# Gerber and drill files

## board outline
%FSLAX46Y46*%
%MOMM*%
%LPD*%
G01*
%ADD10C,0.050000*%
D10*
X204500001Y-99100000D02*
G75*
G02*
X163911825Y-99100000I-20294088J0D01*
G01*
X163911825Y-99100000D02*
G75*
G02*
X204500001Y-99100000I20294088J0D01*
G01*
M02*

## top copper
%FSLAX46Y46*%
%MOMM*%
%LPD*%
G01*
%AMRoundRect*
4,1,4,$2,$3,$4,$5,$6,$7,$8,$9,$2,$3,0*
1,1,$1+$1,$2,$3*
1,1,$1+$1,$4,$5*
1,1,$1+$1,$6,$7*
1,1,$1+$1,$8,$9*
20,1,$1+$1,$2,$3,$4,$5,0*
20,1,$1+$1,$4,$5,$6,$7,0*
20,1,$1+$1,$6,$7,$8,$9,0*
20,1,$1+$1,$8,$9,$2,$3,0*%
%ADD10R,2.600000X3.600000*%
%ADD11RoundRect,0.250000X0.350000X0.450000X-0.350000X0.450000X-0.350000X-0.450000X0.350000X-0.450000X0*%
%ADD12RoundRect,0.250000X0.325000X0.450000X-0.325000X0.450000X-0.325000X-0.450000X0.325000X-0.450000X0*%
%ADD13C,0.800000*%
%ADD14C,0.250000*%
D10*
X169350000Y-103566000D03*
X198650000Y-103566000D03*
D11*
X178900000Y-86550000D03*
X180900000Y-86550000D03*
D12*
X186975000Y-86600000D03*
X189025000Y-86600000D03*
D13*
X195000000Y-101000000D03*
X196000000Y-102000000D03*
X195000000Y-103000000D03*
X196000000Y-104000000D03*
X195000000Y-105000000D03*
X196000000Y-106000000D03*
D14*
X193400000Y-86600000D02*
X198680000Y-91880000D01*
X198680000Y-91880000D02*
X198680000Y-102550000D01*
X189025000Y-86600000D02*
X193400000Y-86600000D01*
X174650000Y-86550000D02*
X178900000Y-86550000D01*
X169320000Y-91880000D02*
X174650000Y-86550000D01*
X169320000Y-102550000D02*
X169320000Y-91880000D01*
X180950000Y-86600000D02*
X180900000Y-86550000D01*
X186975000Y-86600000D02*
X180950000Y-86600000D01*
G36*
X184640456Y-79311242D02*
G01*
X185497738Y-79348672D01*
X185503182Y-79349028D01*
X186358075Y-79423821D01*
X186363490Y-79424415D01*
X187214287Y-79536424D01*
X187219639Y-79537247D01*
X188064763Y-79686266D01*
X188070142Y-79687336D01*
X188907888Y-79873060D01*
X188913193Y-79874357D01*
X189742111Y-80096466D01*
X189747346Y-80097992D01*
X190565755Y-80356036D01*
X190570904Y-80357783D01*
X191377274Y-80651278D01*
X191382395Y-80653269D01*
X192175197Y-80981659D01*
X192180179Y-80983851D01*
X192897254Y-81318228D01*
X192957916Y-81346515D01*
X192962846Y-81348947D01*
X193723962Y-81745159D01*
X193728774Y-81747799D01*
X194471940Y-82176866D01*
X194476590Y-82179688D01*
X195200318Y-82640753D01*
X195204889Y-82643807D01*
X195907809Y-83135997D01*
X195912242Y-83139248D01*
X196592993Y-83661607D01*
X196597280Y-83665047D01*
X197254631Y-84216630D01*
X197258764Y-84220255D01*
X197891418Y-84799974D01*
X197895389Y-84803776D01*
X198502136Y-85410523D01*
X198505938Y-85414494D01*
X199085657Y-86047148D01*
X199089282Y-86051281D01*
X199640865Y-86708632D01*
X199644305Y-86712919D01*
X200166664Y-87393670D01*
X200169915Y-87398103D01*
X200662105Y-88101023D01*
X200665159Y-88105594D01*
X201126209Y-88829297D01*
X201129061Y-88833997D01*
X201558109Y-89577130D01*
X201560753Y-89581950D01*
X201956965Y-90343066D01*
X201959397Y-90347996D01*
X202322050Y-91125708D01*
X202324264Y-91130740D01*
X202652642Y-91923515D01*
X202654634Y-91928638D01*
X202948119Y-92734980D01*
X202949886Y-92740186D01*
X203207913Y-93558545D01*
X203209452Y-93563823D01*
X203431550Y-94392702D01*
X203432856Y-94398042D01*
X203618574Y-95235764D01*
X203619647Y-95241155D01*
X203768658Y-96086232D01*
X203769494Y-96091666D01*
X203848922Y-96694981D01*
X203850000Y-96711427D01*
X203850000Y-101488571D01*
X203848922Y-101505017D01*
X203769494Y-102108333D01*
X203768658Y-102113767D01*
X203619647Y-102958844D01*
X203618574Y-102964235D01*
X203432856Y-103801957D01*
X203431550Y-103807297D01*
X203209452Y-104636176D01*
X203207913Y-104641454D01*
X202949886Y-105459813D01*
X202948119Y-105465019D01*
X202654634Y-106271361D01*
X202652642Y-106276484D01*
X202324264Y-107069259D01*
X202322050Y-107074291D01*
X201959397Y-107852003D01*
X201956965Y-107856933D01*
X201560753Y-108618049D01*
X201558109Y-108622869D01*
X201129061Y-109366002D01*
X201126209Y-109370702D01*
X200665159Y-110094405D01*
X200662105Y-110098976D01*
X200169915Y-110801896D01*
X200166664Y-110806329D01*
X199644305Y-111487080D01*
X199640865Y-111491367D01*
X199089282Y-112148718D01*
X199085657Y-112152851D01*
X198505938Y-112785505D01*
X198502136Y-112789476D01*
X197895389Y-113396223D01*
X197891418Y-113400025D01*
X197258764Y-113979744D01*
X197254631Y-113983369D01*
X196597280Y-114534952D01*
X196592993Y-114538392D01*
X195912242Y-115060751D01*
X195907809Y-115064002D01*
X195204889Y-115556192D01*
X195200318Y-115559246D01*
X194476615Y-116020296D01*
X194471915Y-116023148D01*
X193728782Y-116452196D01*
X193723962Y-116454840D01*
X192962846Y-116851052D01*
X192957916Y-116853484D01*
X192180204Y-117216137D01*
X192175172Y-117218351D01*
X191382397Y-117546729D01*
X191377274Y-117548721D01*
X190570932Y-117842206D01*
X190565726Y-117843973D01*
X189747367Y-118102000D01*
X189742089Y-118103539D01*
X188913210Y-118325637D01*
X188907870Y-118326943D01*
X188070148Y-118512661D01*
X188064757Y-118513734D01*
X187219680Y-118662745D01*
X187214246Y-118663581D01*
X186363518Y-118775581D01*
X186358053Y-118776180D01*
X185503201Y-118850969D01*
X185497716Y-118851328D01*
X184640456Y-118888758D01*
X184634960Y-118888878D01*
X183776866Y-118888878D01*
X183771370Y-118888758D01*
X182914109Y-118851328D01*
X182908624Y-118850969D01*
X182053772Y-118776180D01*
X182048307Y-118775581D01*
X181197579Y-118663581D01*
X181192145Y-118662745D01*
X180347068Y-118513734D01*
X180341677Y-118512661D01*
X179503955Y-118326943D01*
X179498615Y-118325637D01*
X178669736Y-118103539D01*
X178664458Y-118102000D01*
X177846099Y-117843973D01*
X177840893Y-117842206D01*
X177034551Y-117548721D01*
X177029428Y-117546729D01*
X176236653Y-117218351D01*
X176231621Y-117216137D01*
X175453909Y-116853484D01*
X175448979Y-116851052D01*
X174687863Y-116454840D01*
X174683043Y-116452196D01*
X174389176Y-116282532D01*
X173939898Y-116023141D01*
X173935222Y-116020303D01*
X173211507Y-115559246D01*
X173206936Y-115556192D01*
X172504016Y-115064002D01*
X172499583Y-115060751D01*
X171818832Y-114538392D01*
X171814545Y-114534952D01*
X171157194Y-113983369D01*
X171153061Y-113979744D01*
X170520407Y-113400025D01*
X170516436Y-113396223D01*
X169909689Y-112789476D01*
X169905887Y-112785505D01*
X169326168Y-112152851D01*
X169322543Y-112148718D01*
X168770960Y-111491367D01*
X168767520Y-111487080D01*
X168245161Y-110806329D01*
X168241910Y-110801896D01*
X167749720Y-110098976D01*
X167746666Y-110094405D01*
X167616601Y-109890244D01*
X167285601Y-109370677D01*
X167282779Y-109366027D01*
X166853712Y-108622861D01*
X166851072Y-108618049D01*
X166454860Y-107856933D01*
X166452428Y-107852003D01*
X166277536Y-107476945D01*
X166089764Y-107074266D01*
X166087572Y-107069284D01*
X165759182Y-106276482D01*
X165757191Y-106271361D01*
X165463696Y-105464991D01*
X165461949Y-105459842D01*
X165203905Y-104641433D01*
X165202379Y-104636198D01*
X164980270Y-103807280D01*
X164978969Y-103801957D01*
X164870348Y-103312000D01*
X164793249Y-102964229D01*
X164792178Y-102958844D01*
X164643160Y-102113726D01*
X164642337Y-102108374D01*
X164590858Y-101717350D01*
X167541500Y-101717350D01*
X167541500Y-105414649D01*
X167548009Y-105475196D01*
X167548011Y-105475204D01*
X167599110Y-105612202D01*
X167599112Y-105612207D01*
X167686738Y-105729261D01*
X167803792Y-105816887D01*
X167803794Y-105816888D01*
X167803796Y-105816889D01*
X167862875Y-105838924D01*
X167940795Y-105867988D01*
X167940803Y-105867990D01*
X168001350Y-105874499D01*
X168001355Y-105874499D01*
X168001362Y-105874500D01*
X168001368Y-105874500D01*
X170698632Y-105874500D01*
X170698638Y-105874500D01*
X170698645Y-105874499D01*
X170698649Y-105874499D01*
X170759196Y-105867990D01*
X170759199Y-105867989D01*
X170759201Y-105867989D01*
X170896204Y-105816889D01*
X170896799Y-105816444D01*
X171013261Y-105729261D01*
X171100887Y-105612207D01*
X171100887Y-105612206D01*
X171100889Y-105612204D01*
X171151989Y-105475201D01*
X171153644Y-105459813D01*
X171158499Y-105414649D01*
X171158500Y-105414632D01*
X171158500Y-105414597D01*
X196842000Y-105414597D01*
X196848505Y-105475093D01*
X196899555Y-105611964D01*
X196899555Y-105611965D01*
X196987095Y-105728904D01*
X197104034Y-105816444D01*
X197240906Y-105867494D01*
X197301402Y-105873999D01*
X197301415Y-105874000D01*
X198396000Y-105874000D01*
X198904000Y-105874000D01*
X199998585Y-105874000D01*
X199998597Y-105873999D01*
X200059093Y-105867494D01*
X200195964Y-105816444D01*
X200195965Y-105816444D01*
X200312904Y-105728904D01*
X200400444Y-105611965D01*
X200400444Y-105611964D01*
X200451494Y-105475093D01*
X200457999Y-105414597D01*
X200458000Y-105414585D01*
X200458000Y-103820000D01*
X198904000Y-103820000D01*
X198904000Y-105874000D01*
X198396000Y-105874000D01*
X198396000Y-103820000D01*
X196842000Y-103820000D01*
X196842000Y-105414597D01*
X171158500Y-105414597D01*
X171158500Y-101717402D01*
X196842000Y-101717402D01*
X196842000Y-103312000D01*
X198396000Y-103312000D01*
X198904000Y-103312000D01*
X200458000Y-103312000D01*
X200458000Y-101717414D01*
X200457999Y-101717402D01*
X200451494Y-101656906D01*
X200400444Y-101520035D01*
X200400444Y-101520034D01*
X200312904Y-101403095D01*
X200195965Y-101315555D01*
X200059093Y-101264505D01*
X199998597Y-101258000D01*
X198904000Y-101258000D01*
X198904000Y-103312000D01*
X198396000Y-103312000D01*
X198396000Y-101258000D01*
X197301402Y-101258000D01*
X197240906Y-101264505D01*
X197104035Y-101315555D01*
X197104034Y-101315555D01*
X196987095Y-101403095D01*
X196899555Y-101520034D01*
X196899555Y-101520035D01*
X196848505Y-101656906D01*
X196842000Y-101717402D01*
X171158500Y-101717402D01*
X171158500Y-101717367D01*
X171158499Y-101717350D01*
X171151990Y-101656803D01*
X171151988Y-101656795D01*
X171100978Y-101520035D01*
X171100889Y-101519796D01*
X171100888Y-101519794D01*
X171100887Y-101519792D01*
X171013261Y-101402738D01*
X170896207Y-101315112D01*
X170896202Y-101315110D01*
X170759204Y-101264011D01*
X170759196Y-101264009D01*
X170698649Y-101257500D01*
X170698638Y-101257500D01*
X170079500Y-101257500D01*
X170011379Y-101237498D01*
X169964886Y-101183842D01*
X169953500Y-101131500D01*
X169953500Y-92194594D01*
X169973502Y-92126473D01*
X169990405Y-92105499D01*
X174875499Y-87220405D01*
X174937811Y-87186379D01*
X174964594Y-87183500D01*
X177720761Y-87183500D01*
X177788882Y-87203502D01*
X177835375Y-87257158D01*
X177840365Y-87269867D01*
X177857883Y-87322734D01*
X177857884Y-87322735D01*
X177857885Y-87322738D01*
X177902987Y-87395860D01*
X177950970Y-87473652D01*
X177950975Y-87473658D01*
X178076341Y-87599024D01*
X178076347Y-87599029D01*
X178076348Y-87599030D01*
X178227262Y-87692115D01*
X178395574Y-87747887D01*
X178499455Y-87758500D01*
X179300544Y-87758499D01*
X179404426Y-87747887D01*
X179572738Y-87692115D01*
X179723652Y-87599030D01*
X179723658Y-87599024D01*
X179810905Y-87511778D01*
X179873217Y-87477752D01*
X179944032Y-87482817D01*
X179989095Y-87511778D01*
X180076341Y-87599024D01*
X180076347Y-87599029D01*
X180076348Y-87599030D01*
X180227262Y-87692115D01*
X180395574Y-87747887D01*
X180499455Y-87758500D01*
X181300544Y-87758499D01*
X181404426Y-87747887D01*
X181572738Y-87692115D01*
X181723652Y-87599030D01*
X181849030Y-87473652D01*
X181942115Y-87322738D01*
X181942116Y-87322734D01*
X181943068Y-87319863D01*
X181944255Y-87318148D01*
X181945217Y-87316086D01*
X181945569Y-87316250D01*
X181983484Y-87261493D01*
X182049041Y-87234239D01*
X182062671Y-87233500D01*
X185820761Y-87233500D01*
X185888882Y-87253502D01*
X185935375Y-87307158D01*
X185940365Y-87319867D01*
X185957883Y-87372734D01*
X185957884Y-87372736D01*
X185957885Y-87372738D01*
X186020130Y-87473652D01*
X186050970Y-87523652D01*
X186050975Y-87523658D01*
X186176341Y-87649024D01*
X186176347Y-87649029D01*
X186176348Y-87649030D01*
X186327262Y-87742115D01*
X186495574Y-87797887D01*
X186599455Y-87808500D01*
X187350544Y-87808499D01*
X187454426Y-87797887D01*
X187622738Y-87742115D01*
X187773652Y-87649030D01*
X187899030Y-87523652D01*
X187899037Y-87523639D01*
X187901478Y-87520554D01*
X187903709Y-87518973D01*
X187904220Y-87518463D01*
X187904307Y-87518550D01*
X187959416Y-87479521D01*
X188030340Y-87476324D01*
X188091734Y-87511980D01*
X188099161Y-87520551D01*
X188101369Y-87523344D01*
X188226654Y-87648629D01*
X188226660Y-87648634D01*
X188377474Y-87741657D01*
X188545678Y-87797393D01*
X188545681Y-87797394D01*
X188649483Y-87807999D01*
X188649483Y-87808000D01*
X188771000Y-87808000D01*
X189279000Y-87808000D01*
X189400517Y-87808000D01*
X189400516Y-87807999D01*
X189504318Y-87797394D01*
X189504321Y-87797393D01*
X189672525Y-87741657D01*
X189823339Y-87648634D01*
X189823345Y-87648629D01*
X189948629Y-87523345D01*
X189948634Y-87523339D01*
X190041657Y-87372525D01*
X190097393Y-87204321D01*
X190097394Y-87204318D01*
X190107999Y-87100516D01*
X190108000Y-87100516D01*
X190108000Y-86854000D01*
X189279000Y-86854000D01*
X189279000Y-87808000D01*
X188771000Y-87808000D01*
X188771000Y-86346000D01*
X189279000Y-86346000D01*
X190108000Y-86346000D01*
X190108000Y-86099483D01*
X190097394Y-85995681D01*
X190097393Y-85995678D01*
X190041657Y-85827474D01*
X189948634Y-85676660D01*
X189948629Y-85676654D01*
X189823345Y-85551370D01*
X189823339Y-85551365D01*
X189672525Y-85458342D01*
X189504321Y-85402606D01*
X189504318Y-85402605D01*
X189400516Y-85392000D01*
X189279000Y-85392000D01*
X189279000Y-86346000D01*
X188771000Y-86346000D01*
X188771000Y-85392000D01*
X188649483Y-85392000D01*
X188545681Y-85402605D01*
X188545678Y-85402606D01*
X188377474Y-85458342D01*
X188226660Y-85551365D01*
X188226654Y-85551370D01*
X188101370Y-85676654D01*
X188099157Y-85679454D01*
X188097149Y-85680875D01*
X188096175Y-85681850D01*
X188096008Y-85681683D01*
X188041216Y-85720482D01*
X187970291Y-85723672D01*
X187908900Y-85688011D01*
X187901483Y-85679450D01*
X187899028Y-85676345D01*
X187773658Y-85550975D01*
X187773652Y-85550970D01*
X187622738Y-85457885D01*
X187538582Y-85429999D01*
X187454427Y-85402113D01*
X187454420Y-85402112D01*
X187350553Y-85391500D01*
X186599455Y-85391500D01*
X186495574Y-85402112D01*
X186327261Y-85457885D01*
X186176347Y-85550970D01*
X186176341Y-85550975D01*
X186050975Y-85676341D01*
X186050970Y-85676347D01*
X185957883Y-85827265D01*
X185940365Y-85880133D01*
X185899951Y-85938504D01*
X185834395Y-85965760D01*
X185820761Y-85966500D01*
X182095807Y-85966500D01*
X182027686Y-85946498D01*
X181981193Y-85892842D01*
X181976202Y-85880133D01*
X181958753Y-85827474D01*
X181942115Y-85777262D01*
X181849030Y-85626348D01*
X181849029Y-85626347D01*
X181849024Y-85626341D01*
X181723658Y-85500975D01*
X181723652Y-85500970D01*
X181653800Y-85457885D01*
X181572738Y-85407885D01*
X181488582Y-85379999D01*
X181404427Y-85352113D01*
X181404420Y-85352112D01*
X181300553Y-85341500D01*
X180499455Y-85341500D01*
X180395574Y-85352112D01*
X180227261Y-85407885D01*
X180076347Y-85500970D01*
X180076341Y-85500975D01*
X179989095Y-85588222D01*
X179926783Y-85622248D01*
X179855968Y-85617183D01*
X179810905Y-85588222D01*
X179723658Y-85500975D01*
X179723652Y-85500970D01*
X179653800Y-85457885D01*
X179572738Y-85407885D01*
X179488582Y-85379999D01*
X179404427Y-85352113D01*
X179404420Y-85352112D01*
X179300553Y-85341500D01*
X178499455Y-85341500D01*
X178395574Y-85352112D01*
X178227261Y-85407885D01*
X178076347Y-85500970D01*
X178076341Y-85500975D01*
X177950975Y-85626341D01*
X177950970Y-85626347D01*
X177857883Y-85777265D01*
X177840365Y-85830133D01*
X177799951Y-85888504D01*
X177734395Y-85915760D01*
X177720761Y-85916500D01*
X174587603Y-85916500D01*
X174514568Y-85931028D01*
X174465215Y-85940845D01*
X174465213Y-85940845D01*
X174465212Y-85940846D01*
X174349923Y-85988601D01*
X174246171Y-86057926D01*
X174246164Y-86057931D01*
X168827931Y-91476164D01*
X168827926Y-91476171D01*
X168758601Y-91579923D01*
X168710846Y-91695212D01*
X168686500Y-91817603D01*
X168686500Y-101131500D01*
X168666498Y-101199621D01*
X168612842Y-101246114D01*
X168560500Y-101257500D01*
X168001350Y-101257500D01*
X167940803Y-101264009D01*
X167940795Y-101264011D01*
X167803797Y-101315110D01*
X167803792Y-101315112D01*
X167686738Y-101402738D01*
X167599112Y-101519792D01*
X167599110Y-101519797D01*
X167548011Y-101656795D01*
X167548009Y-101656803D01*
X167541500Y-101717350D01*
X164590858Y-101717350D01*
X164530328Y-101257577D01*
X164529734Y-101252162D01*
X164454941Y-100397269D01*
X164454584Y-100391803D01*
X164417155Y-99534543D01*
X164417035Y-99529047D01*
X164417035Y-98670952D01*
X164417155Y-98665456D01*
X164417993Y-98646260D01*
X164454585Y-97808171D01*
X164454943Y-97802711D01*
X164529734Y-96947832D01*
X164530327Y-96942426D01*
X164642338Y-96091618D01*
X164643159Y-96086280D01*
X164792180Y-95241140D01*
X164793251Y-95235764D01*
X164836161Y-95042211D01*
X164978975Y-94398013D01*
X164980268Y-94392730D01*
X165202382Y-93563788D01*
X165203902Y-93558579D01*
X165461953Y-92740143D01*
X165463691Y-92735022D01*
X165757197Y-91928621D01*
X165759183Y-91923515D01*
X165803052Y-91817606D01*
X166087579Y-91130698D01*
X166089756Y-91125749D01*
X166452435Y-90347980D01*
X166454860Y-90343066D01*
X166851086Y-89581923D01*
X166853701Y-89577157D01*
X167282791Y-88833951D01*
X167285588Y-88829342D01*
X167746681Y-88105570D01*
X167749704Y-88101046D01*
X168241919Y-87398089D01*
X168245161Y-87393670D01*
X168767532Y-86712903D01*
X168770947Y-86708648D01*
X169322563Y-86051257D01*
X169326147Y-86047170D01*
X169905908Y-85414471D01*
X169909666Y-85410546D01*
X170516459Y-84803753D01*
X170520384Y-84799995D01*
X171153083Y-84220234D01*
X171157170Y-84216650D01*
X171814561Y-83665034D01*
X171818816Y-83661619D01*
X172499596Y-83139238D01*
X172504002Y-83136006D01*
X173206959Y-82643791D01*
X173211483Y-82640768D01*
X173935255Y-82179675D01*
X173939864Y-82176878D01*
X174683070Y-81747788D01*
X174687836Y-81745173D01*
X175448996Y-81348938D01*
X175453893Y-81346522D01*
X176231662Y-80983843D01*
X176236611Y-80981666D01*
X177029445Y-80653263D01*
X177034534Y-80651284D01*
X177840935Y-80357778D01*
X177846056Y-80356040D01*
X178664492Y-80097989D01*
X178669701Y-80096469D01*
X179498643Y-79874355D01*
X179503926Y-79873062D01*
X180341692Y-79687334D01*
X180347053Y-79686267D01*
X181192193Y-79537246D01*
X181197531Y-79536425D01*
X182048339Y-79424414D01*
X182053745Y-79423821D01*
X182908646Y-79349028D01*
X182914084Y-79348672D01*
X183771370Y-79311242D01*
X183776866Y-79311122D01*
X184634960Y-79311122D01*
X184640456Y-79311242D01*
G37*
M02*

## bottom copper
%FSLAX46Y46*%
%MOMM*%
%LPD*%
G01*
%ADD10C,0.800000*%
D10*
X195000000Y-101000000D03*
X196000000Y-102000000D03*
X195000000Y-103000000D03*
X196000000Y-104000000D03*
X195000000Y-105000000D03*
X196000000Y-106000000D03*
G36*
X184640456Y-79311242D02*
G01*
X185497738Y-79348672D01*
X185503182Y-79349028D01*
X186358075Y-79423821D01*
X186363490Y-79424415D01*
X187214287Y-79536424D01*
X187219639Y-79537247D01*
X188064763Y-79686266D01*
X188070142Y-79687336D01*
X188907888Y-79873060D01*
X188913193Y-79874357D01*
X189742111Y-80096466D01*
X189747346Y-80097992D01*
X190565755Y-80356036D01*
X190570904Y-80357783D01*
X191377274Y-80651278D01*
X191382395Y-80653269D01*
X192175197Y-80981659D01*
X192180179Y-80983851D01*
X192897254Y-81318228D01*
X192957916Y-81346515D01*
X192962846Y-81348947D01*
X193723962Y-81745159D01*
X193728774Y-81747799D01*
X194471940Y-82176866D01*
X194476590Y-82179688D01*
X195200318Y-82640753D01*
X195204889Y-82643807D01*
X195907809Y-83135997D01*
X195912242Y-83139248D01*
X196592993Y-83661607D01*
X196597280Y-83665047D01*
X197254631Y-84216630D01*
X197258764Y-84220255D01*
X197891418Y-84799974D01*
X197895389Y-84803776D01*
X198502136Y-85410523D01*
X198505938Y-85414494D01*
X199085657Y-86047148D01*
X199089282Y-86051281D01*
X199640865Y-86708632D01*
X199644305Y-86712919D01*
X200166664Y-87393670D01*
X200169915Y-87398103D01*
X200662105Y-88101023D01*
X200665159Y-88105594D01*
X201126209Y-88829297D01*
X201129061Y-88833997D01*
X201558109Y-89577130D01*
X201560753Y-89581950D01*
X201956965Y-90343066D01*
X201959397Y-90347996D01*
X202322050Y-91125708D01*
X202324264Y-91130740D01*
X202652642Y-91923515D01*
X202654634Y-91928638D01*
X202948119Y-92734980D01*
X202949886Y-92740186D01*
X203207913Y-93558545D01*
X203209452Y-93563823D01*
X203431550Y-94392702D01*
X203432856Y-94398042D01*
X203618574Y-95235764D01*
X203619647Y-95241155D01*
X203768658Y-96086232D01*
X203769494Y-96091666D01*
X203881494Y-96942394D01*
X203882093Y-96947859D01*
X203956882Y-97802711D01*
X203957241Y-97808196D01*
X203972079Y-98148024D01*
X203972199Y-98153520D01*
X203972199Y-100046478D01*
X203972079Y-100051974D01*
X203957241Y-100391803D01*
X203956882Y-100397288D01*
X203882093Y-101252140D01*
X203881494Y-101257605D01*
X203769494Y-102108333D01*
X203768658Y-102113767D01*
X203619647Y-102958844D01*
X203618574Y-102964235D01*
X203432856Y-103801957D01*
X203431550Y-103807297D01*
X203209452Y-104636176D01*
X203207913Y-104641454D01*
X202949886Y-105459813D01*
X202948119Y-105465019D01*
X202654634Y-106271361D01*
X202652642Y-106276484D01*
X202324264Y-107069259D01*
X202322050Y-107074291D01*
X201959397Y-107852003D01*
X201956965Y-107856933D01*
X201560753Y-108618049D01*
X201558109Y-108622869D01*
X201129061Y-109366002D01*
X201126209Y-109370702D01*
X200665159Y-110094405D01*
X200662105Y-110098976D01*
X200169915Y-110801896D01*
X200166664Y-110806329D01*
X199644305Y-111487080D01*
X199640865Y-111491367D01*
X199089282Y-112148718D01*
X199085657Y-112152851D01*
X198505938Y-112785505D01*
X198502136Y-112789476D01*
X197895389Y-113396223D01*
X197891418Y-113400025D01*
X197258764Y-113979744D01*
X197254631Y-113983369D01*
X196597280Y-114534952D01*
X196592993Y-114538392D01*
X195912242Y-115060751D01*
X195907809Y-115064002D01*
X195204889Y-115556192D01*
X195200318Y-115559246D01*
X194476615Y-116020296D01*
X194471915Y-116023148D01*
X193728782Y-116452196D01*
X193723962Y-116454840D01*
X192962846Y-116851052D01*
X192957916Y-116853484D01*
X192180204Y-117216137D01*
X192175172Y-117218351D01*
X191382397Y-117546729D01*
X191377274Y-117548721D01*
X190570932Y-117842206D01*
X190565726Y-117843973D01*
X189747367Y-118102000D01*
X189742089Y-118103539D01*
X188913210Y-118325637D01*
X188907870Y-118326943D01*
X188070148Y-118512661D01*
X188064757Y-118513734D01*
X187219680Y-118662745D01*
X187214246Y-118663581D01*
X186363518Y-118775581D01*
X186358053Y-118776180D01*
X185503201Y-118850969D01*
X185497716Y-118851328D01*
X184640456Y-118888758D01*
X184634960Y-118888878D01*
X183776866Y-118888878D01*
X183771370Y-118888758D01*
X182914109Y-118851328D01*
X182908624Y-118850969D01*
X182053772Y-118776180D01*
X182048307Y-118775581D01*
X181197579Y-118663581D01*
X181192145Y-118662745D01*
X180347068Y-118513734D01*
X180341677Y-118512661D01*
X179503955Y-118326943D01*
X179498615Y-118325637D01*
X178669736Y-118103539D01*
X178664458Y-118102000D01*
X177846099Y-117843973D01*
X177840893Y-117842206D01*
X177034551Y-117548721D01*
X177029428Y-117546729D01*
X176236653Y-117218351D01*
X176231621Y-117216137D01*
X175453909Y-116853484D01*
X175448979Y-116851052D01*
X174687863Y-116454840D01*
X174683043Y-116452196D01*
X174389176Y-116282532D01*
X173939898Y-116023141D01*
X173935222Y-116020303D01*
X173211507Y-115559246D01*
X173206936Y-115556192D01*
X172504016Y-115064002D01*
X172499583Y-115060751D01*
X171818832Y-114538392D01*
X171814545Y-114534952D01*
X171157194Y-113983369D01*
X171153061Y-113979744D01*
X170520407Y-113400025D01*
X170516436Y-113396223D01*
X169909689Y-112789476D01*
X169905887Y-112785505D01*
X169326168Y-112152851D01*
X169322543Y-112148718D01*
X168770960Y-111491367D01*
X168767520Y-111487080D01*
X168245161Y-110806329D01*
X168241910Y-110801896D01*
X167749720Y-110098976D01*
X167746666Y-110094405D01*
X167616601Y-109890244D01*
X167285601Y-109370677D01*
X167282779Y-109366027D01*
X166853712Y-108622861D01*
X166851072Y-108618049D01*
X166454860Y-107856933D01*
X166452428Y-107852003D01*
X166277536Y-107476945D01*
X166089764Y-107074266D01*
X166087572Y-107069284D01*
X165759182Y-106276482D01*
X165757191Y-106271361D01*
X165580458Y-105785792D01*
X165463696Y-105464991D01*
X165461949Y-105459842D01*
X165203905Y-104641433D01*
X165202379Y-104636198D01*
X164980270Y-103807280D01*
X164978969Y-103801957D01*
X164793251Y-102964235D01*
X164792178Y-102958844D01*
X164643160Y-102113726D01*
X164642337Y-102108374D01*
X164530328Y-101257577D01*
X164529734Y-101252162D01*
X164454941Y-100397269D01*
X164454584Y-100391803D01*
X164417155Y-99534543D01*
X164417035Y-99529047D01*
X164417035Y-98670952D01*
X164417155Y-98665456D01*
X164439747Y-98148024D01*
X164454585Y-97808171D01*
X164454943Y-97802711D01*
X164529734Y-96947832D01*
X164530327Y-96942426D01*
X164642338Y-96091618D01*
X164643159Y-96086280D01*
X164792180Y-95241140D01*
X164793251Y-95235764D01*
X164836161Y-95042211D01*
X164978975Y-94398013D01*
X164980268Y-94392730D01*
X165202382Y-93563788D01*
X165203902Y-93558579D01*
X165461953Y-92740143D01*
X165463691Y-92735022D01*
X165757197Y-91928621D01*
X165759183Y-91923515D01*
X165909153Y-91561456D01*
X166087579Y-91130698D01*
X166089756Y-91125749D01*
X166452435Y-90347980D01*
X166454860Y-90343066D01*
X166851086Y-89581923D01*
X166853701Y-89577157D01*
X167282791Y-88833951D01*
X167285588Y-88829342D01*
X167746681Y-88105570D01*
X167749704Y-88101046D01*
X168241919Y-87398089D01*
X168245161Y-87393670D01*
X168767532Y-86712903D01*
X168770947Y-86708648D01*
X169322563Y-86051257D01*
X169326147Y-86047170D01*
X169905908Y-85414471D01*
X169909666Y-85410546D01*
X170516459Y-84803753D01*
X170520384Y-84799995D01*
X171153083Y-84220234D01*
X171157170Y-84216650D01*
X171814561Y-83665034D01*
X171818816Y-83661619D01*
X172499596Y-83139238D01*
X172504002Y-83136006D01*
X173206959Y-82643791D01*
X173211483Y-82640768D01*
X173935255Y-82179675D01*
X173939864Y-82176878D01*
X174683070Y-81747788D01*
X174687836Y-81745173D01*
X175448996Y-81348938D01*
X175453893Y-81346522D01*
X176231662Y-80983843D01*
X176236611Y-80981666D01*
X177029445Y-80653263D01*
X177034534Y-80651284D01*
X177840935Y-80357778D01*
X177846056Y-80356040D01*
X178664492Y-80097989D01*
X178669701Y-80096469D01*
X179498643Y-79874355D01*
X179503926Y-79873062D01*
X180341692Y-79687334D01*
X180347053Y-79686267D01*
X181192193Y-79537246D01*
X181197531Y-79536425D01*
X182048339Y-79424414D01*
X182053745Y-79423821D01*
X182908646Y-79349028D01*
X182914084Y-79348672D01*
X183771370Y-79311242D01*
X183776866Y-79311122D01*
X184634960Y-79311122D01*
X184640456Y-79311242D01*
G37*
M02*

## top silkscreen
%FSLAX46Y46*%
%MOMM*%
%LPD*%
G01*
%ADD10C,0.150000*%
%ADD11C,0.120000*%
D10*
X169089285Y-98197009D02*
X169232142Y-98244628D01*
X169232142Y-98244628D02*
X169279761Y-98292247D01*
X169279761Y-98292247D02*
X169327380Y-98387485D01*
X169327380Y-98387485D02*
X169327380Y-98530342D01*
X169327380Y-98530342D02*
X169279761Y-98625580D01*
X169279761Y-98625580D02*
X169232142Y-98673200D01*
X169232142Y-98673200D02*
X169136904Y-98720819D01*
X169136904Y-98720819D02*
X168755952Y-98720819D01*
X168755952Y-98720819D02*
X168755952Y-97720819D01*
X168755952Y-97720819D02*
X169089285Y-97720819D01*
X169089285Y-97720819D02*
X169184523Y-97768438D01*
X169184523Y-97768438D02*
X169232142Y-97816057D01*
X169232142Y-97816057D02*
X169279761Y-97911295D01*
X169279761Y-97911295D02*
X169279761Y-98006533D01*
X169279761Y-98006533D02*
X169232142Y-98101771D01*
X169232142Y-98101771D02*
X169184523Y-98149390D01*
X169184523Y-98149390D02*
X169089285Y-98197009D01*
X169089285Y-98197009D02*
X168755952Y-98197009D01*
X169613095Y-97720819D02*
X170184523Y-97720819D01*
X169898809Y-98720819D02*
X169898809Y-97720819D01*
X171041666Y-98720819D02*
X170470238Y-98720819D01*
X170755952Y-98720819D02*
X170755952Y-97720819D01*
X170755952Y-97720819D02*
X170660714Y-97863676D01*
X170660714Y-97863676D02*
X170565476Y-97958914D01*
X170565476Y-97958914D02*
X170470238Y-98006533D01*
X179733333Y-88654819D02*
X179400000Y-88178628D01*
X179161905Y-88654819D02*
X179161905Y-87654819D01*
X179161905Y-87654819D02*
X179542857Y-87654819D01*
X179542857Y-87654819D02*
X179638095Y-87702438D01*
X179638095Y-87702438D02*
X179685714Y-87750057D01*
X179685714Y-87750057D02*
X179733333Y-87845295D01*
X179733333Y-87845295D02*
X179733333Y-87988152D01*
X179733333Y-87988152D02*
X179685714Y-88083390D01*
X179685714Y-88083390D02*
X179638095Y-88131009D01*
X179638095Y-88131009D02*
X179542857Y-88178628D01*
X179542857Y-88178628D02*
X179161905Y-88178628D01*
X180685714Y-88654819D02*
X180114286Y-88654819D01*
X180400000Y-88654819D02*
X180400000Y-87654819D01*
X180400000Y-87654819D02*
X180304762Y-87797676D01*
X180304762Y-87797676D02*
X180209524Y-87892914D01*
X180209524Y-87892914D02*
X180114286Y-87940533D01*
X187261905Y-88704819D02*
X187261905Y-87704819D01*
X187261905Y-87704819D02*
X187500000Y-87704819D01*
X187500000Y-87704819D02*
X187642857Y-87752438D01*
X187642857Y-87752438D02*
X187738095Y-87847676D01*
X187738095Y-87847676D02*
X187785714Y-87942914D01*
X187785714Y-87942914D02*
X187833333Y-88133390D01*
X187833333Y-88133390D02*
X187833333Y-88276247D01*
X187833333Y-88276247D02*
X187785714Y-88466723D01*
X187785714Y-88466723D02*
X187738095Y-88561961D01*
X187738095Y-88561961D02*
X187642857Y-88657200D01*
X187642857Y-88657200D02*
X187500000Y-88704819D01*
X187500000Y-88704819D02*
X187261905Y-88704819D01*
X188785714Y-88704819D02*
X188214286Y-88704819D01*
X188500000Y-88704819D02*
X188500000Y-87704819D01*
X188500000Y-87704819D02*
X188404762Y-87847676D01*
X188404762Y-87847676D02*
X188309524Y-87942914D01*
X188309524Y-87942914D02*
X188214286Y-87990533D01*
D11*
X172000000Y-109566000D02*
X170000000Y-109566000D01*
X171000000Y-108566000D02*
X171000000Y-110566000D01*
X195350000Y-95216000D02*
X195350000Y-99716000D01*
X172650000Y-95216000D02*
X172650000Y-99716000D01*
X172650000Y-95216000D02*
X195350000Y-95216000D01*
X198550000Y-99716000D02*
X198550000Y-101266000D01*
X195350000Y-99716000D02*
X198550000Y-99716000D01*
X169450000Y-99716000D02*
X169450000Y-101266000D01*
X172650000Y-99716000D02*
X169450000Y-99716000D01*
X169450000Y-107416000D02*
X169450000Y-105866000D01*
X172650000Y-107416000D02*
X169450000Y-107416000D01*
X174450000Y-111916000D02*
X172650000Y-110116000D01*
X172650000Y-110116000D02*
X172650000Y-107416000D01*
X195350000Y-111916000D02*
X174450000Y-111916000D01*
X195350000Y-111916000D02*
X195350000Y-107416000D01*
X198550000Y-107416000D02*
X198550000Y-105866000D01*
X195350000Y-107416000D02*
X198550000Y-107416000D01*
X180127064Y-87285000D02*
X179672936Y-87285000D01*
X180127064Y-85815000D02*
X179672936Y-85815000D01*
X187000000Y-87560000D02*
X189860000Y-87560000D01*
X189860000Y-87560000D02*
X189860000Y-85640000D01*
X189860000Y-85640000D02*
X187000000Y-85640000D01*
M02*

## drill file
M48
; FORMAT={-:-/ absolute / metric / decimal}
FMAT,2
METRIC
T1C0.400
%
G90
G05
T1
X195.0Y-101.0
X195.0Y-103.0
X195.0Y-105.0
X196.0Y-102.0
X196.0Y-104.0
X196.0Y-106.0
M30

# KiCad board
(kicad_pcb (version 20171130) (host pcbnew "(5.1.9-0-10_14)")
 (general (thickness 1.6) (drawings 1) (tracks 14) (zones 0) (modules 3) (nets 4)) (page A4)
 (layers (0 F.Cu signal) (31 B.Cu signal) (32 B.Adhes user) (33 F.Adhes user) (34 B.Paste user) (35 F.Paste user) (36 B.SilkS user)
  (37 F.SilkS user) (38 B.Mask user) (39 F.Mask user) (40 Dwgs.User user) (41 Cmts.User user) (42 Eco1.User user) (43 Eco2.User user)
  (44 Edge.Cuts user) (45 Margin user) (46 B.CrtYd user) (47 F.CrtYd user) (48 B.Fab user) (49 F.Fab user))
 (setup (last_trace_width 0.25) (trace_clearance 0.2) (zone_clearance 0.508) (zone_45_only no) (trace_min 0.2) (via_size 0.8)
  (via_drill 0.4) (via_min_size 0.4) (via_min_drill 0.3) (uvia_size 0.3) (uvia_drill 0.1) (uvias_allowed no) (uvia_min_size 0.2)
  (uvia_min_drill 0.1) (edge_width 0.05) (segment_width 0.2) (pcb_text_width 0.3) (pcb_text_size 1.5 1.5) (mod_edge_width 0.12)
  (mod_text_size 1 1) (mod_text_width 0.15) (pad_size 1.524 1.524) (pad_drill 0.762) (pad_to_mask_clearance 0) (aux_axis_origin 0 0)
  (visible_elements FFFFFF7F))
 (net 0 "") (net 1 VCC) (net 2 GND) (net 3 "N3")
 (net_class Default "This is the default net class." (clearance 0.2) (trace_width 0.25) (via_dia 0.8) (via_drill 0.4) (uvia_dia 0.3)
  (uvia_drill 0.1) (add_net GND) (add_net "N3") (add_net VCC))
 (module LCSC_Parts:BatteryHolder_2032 (layer F.Cu) (at 184 102.55 180)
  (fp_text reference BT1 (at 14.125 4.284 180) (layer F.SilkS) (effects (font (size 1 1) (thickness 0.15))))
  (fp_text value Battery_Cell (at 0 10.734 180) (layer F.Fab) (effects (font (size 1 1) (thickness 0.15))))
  (fp_line (start 12 -7.016) (end 14 -7.016) (layer F.SilkS) (width 0.12))
  (fp_line (start 13 -6.016) (end 13 -8.016) (layer F.SilkS) (width 0.12))
  (fp_line (start -11.35 7.334) (end -11.35 2.834) (layer F.SilkS) (width 0.12))
  (fp_line (start 11.35 7.334) (end 11.35 2.834) (layer F.SilkS) (width 0.12))
  (fp_line (start 11.35 7.334) (end -11.35 7.334) (layer F.SilkS) (width 0.12))
  (fp_line (start -14.55 2.834) (end -14.55 1.284) (layer F.SilkS) (width 0.12))
  (fp_line (start -11.35 2.834) (end -14.55 2.834) (layer F.SilkS) (width 0.12))
  (fp_line (start 14.55 2.834) (end 14.55 1.284) (layer F.SilkS) (width 0.12))
  (fp_line (start 11.35 2.834) (end 14.55 2.834) (layer F.SilkS) (width 0.12))
  (fp_line (start 14.55 -4.866) (end 14.55 -3.316) (layer F.SilkS) (width 0.12))
  (fp_line (start 11.35 -4.866) (end 14.55 -4.866) (layer F.SilkS) (width 0.12))
  (fp_line (start 9.55 -9.366) (end 11.35 -7.566) (layer F.SilkS) (width 0.12))
  (fp_line (start 11.35 -7.566) (end 11.35 -4.866) (layer F.SilkS) (width 0.12))
  (fp_line (start -11.35 -9.366) (end 9.55 -9.366) (layer F.SilkS) (width 0.12))
  (fp_line (start -11.35 -9.366) (end -11.35 -4.866) (layer F.SilkS) (width 0.12))
  (fp_line (start -14.55 -4.866) (end -14.55 -3.316) (layer F.SilkS) (width 0.12))
  (fp_line (start -11.35 -4.866) (end -14.55 -4.866) (layer F.SilkS) (width 0.12))
  (pad 1 smd rect (at 14.65 -1.016 180) (size 2.6 3.6) (layers F.Cu F.Paste F.Mask) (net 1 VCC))
  (pad 2 smd rect (at -14.65 -1.016 180) (size 2.6 3.6) (layers F.Cu F.Paste F.Mask) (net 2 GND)))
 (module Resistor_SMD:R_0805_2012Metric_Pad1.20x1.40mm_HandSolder (layer F.Cu) (at 179.9 86.55 180)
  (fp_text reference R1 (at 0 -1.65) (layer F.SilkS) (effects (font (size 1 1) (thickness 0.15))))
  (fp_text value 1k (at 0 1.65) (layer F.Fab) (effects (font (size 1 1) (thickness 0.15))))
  (fp_line (start -0.227064 -0.735) (end 0.227064 -0.735) (layer F.SilkS) (width 0.12))
  (fp_line (start -0.227064 0.735) (end 0.227064 0.735) (layer F.SilkS) (width 0.12))
  (pad 2 smd roundrect (at 1 0 180) (size 1.2 1.4) (layers F.Cu F.Paste F.Mask) (roundrect_rratio 0.208333) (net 1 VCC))
  (pad 1 smd roundrect (at -1 0 180) (size 1.2 1.4) (layers F.Cu F.Paste F.Mask) (roundrect_rratio 0.208333) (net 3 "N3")))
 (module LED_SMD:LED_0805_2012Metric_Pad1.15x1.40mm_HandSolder (layer F.Cu) (at 188 86.6 180)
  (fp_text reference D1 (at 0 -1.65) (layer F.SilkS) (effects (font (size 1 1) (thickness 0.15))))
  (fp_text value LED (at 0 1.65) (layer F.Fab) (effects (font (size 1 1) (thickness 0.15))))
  (fp_line (start 1 -0.96) (end -1.86 -0.96) (layer F.SilkS) (width 0.12))
  (fp_line (start -1.86 -0.96) (end -1.86 0.96) (layer F.SilkS) (width 0.12))
  (fp_line (start -1.86 0.96) (end 1 0.96) (layer F.SilkS) (width 0.12))
  (pad 2 smd roundrect (at 1.025 0 180) (size 1.15 1.4) (layers F.Cu F.Paste F.Mask) (roundrect_rratio 0.217391) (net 3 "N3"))
  (pad 1 smd roundrect (at -1.025 0 180) (size 1.15 1.4) (layers F.Cu F.Paste F.Mask) (roundrect_rratio 0.217391) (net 2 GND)))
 (gr_circle (center 184.205913 99.1) (end 198.505913 84.7) (layer Edge.Cuts) (width 0.05))
 (segment (start 193.4 86.6) (end 198.68 91.88) (width 0.25) (layer F.Cu) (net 2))
 (segment (start 198.68 91.88) (end 198.68 102.55) (width 0.25) (layer F.Cu) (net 2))
 (segment (start 189.025 86.6) (end 193.4 86.6) (width 0.25) (layer F.Cu) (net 2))
 (segment (start 174.65 86.55) (end 178.9 86.55) (width 0.25) (layer F.Cu) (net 1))
 (segment (start 169.32 91.88) (end 174.65 86.55) (width 0.25) (layer F.Cu) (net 1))
 (segment (start 169.32 102.55) (end 169.32 91.88) (width 0.25) (layer F.Cu) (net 1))
 (segment (start 180.95 86.6) (end 180.9 86.55) (width 0.25) (layer F.Cu) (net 3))
 (segment (start 186.975 86.6) (end 180.95 86.6) (width 0.25) (layer F.Cu) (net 3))
 (via (at 195 101) (size 0.8) (drill 0.4) (layers F.Cu B.Cu) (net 2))
 (via (at 196 102) (size 0.8) (drill 0.4) (layers F.Cu B.Cu) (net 2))
 (via (at 195 103) (size 0.8) (drill 0.4) (layers F.Cu B.Cu) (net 2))
 (via (at 196 104) (size 0.8) (drill 0.4) (layers F.Cu B.Cu) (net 2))
 (via (at 195 105) (size 0.8) (drill 0.4) (layers F.Cu B.Cu) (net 2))
 (via (at 196 106) (size 0.8) (drill 0.4) (layers F.Cu B.Cu) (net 2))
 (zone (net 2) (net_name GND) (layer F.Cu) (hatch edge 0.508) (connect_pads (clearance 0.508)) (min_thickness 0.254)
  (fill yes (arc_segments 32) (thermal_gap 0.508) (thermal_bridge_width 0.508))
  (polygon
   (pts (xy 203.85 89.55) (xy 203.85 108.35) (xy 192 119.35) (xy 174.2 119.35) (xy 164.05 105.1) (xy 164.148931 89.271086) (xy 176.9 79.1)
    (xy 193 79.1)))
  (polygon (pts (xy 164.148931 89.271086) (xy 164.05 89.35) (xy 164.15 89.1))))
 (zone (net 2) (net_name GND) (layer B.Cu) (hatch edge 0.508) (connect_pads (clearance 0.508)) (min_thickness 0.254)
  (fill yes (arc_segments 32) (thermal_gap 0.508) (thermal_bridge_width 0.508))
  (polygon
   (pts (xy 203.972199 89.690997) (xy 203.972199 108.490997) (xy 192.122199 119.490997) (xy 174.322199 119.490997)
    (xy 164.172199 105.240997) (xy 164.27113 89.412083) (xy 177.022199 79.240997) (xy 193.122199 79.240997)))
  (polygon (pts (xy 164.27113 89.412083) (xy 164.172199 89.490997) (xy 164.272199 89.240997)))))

